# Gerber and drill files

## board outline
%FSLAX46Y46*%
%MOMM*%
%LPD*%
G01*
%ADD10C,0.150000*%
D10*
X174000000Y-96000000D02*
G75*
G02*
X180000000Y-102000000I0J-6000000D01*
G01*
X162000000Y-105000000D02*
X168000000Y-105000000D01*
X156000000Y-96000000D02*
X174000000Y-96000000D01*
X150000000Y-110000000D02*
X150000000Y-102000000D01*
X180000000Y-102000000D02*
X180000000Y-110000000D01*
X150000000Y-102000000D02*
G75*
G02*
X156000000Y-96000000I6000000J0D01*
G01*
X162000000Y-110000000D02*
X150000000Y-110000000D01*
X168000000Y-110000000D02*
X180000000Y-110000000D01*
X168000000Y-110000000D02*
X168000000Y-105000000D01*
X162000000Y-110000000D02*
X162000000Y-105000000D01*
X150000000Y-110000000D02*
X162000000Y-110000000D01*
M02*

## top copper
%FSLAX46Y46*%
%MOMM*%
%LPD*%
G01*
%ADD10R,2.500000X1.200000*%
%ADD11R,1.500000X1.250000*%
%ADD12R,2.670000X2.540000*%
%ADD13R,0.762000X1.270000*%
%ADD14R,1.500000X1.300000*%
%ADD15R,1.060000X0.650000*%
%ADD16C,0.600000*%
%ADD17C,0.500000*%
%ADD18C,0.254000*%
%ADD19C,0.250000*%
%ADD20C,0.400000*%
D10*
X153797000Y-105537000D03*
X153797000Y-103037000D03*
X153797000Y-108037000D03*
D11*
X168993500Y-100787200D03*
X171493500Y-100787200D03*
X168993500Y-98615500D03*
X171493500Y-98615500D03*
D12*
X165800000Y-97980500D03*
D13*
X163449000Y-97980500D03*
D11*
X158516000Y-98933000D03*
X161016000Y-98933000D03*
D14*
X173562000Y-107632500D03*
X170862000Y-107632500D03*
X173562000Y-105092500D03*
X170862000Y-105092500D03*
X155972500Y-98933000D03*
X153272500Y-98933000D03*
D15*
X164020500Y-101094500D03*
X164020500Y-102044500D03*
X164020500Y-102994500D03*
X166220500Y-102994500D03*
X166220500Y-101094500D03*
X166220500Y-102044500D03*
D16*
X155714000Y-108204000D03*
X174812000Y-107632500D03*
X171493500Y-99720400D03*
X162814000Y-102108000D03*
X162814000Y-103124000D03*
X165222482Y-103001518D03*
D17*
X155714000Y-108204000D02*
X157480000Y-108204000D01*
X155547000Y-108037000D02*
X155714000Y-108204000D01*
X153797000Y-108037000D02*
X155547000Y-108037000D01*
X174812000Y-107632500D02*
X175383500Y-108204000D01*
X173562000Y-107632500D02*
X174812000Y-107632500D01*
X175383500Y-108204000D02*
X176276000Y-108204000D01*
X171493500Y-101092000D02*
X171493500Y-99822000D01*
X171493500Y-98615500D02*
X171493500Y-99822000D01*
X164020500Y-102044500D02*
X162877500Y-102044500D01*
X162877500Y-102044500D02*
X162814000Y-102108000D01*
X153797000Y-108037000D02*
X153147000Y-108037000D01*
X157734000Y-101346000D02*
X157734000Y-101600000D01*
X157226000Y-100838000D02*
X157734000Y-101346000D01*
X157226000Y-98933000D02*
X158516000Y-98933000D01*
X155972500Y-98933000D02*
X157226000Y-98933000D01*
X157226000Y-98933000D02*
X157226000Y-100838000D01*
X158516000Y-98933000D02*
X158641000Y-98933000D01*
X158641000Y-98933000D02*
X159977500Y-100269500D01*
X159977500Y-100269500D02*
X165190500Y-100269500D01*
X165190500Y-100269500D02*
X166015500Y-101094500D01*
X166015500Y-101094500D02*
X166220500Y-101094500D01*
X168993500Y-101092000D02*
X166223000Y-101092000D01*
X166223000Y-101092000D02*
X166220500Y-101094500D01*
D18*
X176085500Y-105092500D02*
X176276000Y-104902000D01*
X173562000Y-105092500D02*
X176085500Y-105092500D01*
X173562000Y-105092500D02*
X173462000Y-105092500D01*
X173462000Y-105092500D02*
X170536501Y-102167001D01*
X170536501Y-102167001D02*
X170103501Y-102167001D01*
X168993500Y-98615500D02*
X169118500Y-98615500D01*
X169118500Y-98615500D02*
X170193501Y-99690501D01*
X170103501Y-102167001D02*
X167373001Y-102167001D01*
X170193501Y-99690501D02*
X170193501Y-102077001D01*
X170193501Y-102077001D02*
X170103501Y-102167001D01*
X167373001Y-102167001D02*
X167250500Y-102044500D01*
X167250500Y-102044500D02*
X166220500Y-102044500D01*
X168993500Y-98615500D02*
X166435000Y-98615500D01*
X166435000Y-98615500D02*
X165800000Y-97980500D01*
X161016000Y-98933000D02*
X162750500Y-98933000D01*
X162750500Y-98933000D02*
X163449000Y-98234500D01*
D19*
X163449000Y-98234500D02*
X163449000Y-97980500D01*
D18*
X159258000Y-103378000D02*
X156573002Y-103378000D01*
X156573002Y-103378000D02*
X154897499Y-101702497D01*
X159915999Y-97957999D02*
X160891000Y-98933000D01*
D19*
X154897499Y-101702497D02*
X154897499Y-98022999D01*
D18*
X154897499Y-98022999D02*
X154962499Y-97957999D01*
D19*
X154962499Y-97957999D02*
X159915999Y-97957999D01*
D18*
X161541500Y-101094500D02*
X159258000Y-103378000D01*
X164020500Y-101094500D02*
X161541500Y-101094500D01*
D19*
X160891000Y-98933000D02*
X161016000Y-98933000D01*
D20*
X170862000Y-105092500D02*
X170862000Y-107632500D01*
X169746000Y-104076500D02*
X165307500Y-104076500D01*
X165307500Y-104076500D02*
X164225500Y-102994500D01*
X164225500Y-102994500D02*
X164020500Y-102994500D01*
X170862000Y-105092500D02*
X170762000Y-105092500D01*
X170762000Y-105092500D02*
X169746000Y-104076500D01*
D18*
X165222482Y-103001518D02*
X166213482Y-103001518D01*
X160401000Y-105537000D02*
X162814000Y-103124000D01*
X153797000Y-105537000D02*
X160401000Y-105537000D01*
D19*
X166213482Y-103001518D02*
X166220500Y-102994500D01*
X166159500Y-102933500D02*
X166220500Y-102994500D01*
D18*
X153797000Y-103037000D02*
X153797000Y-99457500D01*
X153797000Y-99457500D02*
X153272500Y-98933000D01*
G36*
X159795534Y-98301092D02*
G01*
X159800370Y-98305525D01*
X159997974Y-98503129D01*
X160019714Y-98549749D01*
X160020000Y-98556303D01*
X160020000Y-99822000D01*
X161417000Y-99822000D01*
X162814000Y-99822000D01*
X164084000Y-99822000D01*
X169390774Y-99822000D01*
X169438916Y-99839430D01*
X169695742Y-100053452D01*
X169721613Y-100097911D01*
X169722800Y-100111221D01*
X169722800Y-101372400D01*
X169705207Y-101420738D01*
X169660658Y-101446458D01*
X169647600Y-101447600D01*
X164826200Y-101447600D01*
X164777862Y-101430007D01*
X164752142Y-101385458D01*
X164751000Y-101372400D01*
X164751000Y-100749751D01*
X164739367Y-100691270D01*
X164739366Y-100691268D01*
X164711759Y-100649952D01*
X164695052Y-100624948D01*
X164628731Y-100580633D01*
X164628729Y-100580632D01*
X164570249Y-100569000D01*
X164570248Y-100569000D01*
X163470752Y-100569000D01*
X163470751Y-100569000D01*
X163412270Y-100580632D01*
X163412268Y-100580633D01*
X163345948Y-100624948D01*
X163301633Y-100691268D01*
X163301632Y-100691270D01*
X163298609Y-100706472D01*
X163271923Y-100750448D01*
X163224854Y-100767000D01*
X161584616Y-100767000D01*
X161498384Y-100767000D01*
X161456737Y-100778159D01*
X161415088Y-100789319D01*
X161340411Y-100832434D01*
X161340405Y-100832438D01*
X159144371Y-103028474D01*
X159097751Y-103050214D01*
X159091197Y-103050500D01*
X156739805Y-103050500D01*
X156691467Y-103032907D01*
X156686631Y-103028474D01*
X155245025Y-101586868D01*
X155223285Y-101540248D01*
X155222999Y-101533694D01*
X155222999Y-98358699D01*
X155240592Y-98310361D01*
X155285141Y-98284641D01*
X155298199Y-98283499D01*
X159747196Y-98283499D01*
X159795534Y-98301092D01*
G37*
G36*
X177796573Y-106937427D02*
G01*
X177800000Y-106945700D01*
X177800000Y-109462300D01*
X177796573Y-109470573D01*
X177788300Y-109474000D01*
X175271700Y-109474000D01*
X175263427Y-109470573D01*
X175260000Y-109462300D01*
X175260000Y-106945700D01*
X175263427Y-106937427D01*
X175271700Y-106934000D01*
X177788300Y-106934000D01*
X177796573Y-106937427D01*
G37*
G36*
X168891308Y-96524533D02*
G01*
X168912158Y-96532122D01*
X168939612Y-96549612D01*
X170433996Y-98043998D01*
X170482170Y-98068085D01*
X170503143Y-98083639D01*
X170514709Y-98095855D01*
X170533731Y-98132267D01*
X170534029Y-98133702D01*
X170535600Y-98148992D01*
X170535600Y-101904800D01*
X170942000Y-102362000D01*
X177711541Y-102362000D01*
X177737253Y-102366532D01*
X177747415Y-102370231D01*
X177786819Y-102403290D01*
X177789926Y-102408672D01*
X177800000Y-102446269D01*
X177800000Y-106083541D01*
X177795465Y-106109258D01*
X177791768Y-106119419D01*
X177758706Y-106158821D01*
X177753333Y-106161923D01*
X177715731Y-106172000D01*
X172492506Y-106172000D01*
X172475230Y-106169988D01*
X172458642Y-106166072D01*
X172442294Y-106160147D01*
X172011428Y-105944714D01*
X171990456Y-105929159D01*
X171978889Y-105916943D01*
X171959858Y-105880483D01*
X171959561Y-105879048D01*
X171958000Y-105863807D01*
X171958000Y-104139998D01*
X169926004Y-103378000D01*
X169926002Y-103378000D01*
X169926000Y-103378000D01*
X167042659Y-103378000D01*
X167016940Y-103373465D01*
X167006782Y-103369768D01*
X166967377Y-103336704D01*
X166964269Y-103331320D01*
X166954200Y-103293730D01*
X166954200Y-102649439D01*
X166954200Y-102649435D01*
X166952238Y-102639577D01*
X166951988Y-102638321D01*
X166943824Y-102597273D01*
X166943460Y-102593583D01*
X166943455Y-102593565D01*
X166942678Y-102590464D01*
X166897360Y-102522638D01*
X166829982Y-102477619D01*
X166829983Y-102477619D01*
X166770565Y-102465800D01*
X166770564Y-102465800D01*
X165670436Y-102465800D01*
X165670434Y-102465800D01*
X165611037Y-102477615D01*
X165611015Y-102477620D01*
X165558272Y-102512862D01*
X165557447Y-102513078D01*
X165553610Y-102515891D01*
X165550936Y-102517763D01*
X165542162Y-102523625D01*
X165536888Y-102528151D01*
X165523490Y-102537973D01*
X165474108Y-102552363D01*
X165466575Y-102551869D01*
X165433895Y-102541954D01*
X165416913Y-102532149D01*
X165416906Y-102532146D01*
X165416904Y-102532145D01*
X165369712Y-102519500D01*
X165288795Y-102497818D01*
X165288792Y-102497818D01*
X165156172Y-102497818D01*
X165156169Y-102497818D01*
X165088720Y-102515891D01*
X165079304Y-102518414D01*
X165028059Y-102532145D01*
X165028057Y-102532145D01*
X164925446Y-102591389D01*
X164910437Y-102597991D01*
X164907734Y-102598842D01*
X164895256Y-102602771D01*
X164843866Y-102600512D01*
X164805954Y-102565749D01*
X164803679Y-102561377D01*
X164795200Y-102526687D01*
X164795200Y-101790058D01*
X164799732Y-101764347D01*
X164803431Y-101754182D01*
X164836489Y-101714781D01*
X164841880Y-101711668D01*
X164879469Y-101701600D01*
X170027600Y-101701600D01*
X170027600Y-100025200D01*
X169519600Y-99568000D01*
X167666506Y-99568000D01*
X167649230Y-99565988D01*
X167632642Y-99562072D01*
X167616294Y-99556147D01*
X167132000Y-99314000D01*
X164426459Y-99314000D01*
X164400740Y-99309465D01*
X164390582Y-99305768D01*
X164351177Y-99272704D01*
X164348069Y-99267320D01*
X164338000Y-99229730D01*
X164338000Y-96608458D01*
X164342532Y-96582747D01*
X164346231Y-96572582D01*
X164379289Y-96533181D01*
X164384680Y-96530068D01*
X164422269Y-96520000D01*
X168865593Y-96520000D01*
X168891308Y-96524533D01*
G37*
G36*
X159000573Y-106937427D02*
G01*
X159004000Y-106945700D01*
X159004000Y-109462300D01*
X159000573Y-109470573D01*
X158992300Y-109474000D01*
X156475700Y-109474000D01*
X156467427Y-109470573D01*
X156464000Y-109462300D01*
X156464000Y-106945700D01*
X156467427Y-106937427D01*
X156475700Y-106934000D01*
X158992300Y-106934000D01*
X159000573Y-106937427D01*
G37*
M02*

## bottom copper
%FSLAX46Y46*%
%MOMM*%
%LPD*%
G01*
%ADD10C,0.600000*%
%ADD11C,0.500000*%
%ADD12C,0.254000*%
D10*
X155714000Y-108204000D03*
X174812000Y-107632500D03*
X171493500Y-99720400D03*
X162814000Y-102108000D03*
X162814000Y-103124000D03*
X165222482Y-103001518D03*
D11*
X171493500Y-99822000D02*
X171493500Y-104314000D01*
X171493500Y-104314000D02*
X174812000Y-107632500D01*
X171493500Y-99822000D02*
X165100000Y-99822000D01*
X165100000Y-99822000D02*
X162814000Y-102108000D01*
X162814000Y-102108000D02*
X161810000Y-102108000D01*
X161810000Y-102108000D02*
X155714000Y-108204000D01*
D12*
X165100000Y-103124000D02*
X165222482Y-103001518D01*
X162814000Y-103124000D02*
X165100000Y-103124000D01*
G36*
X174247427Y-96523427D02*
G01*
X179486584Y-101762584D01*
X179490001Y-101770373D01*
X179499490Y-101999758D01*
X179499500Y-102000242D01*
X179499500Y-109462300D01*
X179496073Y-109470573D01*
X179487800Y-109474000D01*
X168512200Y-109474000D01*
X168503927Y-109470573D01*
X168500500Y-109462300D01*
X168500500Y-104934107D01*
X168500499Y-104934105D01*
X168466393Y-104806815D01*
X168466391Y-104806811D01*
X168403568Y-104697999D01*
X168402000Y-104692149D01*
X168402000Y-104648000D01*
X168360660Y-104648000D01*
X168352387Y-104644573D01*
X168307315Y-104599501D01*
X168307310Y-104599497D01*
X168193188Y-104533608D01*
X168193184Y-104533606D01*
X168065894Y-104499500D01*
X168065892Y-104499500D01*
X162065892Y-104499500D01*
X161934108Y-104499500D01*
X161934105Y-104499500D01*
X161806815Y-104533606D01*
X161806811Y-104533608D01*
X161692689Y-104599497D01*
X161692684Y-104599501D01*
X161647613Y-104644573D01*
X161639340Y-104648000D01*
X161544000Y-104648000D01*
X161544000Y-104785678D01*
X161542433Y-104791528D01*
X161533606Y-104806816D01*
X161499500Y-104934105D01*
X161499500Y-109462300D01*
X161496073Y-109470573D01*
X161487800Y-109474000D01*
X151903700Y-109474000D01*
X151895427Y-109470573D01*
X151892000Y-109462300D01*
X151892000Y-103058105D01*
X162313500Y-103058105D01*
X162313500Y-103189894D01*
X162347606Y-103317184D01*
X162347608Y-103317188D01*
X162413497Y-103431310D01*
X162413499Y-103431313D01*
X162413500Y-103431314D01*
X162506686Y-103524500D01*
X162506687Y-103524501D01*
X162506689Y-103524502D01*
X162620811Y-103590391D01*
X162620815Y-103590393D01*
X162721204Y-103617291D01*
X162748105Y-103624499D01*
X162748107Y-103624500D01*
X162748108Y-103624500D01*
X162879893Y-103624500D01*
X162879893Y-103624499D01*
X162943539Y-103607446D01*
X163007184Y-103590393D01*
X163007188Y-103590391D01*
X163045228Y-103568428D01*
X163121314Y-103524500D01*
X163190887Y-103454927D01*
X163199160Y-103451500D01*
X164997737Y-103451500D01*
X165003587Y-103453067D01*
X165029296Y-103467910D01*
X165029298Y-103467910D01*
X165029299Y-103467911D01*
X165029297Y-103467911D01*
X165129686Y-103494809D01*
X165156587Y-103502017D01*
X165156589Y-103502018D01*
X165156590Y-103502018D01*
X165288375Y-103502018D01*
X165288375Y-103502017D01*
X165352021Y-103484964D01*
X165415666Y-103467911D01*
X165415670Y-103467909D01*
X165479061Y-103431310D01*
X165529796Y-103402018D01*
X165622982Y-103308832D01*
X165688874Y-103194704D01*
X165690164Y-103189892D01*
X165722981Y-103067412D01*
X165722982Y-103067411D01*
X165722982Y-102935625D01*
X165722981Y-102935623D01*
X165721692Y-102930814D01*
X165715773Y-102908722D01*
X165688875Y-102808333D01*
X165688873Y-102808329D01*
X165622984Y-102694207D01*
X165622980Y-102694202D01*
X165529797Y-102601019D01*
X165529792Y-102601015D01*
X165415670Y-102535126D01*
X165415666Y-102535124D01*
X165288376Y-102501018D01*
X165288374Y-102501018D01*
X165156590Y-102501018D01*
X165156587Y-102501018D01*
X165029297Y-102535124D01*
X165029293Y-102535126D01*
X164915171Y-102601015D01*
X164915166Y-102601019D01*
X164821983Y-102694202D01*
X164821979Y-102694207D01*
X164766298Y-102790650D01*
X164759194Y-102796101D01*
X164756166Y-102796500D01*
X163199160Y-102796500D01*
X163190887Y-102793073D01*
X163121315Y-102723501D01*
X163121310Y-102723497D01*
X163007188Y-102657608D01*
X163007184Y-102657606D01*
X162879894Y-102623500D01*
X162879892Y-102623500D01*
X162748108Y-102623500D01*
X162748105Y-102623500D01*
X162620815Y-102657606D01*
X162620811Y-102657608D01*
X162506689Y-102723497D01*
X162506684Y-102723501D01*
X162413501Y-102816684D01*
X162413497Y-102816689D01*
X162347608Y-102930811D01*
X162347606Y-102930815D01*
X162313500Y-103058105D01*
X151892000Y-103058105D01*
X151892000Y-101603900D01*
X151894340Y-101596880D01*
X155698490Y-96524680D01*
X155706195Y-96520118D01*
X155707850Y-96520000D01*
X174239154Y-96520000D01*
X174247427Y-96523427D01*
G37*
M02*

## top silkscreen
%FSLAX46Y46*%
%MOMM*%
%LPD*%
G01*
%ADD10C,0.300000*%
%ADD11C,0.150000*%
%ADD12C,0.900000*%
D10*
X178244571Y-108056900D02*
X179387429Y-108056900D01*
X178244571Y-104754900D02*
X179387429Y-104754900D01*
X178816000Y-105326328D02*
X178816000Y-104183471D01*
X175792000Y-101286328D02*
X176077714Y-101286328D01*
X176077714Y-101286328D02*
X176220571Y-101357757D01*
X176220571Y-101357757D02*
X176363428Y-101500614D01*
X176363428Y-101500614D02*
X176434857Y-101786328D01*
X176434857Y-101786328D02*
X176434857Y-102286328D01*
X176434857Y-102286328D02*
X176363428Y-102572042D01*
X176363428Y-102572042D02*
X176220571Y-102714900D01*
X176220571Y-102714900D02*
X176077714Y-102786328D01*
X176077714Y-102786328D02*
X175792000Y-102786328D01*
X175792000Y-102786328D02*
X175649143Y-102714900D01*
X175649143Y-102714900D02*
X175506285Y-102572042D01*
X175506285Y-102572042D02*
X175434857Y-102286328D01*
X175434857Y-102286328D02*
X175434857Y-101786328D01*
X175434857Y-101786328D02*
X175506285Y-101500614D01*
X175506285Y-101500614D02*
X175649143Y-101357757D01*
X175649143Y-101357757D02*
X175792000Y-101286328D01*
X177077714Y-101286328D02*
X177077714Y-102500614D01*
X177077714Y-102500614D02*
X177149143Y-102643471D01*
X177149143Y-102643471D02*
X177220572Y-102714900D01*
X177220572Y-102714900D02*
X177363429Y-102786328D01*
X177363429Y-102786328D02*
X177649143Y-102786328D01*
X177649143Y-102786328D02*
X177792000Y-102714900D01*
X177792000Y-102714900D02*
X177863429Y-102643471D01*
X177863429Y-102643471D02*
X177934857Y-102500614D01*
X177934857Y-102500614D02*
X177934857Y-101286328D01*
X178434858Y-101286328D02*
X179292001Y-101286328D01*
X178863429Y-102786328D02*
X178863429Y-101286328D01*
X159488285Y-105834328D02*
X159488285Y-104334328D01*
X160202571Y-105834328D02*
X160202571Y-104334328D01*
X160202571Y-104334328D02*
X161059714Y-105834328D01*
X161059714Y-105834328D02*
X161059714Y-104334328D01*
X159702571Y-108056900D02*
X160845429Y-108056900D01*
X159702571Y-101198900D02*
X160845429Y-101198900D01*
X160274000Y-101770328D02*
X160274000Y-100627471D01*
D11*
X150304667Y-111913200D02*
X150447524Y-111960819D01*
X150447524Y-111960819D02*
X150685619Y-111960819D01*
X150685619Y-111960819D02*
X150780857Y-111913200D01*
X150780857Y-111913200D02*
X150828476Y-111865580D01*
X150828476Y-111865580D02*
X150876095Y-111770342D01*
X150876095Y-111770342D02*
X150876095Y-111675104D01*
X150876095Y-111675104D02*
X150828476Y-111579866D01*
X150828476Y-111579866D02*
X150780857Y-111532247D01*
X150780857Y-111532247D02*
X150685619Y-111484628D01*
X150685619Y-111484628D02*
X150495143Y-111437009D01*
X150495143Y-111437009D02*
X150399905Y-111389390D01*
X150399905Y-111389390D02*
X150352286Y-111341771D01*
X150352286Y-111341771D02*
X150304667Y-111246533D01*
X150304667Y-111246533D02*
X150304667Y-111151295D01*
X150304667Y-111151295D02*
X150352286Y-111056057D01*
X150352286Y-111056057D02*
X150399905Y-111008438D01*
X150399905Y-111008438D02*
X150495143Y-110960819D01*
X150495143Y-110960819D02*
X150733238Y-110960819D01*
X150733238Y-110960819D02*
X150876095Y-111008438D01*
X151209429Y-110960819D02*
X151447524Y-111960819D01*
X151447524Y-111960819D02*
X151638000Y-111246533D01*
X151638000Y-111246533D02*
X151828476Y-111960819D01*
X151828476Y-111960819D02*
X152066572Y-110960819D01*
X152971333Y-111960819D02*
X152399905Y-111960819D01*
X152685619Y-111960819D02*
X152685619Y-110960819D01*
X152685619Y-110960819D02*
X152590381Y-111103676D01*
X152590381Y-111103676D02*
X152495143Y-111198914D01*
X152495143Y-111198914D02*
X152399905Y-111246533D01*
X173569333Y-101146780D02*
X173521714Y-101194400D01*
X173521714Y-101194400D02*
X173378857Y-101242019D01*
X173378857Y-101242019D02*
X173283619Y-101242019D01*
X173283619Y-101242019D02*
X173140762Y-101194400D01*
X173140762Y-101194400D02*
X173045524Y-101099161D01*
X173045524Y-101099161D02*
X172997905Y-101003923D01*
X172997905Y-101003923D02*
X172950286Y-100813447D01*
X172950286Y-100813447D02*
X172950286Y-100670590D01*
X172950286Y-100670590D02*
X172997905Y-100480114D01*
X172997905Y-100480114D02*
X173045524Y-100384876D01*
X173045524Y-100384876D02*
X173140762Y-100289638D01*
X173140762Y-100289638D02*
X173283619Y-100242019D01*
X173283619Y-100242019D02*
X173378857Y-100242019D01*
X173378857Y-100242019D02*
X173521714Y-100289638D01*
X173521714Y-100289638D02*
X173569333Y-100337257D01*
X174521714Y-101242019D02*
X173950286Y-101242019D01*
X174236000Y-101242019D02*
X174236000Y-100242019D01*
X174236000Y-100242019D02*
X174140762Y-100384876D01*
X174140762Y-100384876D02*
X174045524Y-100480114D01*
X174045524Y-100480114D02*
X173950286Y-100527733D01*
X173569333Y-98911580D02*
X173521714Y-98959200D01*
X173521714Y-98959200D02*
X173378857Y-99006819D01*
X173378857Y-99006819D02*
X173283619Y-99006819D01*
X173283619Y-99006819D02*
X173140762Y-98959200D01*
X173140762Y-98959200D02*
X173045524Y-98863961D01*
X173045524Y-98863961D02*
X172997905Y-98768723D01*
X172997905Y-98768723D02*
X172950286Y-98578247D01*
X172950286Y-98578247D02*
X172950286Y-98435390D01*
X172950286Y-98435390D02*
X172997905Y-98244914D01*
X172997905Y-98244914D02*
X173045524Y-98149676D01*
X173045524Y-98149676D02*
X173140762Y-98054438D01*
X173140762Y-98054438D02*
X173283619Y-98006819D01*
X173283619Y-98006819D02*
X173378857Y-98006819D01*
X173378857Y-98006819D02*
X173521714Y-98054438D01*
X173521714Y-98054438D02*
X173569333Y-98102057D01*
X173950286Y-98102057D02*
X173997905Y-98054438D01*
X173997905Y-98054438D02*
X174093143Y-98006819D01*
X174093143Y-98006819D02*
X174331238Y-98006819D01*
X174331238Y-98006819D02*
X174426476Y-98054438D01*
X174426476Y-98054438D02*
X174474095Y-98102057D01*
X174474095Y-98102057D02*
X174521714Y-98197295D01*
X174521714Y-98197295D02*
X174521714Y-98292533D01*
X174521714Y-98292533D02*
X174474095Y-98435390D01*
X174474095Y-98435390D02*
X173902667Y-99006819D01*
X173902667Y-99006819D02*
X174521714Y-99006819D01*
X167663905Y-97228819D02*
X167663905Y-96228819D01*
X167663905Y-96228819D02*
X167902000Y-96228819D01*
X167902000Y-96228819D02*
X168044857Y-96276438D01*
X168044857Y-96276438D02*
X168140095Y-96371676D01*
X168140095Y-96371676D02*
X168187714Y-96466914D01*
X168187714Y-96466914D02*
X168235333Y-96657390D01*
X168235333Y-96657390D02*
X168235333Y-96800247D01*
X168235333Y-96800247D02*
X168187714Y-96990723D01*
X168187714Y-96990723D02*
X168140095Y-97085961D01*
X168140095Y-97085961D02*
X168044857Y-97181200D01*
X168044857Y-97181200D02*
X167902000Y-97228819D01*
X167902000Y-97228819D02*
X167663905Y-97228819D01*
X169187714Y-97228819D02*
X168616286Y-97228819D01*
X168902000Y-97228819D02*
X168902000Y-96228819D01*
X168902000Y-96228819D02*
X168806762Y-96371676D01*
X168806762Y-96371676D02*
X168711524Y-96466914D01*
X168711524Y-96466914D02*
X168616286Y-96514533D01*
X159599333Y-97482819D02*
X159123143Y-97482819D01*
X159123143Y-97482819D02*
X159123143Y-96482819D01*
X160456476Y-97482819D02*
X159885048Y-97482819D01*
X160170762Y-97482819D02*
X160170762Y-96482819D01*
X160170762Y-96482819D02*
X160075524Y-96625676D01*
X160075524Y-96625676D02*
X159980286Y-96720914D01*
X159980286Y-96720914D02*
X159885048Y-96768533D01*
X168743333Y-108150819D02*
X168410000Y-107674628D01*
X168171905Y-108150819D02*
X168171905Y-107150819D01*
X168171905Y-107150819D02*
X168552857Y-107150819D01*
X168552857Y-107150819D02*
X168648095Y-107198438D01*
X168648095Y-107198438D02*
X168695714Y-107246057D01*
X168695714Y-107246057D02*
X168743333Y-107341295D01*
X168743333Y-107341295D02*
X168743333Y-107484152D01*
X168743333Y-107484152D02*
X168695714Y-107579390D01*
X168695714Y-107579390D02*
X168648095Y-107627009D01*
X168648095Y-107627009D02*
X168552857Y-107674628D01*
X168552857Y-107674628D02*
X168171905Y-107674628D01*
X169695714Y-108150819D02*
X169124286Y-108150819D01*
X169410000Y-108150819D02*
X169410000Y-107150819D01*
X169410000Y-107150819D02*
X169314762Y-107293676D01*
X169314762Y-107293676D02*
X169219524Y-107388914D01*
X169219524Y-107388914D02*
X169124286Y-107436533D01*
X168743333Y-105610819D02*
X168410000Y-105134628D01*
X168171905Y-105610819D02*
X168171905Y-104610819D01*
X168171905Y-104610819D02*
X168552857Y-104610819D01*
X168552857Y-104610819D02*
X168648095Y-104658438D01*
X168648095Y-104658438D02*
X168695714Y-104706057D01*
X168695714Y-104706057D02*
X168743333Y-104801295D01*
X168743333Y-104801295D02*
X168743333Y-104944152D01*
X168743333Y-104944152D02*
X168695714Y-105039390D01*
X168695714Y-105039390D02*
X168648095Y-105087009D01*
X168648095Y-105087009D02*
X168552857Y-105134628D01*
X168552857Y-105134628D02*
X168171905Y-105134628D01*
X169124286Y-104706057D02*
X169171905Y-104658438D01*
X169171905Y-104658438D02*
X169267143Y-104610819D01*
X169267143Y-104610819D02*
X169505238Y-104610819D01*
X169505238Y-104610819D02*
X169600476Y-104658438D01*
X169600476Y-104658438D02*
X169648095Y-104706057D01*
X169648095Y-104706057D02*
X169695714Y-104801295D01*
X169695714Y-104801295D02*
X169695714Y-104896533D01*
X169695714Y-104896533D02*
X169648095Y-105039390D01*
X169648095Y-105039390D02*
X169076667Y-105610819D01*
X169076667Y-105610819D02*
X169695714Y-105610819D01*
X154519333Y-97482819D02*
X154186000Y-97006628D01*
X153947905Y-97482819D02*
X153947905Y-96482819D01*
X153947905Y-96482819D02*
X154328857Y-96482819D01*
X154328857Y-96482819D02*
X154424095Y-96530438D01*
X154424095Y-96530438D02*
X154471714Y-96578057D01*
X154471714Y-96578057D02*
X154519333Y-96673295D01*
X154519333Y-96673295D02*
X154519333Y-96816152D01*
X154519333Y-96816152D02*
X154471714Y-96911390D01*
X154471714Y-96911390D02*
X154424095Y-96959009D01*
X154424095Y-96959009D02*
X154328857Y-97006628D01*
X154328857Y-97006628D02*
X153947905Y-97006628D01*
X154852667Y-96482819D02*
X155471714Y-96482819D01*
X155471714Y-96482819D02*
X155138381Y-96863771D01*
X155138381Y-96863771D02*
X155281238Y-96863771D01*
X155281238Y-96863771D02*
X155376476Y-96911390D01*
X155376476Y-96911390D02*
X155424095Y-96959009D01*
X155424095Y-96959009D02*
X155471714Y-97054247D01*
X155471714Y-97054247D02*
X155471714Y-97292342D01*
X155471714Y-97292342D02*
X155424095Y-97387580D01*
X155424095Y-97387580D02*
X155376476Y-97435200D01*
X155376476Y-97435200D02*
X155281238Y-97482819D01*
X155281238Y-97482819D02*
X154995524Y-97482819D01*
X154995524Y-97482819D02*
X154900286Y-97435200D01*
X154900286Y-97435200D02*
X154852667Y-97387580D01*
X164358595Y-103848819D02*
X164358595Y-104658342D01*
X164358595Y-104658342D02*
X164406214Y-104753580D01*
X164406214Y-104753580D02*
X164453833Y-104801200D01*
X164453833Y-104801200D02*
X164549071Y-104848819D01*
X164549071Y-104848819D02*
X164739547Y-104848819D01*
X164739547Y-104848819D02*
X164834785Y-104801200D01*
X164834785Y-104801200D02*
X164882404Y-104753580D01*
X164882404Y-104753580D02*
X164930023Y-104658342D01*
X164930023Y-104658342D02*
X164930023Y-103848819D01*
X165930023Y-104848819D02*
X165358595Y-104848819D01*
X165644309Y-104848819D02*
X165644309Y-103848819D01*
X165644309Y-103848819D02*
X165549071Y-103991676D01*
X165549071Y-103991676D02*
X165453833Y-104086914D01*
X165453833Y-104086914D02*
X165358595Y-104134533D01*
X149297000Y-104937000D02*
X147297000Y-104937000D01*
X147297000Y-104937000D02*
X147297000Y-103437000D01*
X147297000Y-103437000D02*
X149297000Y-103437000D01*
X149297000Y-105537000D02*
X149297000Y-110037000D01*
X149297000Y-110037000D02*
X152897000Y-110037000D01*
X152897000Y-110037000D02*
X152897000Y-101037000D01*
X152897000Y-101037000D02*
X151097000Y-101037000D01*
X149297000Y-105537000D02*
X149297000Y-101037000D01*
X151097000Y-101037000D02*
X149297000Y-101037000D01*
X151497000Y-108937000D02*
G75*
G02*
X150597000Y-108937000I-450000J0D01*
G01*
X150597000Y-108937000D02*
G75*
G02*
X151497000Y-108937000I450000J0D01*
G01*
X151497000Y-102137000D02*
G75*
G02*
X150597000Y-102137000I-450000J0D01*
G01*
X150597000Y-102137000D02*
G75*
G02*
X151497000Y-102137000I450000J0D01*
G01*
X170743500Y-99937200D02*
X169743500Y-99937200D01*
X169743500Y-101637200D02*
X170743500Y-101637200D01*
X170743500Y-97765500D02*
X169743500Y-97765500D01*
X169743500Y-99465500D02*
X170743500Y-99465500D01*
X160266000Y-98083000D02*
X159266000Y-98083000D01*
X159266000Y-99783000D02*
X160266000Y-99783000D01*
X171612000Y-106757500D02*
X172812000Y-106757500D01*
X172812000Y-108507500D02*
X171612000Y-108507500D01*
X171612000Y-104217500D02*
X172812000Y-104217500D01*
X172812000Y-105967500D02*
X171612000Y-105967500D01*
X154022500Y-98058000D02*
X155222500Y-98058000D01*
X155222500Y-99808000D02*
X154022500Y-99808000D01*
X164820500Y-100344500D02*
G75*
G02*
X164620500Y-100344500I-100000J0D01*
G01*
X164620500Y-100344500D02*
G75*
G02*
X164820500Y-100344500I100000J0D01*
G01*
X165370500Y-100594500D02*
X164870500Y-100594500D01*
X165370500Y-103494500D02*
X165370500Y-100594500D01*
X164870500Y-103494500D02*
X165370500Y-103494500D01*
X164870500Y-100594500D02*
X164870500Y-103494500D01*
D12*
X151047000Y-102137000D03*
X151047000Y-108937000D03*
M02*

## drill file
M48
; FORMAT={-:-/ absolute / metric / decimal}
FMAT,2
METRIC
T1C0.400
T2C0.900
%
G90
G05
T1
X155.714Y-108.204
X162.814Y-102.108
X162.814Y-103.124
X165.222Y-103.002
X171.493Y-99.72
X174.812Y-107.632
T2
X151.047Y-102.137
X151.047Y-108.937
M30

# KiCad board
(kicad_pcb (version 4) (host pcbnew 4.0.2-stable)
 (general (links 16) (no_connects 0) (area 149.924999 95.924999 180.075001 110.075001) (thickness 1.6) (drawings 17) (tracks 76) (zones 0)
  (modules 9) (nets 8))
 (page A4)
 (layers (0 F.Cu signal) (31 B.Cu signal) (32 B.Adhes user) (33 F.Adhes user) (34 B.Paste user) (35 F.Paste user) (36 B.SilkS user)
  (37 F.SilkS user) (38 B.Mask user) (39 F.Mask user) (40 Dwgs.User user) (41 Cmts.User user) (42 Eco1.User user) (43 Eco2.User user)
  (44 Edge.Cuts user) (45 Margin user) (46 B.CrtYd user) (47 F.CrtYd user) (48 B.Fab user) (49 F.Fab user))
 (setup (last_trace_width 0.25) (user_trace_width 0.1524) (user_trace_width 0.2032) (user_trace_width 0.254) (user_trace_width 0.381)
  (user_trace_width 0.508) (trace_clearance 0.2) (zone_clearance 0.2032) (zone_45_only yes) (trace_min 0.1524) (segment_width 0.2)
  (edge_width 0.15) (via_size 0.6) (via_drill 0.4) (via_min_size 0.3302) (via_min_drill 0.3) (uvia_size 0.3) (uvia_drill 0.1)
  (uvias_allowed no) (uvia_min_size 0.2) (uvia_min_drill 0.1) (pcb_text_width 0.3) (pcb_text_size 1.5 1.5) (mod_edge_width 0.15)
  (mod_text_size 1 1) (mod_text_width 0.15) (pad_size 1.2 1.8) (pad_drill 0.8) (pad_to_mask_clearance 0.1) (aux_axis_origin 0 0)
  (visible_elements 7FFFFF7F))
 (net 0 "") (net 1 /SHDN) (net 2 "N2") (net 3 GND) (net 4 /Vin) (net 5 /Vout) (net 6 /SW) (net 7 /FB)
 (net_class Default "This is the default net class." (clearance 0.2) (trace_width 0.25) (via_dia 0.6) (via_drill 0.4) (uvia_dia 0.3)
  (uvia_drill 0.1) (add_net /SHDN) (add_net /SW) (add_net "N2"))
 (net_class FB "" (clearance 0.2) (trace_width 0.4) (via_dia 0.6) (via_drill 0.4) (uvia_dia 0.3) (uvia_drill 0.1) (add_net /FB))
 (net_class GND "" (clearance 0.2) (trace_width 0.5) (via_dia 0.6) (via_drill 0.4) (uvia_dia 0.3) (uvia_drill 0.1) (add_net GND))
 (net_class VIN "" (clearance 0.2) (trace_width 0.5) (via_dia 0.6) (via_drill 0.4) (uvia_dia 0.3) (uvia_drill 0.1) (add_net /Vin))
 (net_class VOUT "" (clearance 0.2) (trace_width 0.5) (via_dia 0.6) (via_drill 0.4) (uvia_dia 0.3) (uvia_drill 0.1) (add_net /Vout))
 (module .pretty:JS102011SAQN (layer F.Cu) (at 153.797 105.537 270)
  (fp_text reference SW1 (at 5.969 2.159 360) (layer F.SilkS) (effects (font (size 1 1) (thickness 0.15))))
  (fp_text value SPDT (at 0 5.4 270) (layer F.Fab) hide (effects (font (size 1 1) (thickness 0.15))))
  (fp_line (start -0.6 4.5) (end -0.6 6.5) (layer F.SilkS) (width 0.15))
  (fp_line (start -0.6 6.5) (end -2.1 6.5) (layer F.SilkS) (width 0.15))
  (fp_line (start -2.1 6.5) (end -2.1 4.5) (layer F.SilkS) (width 0.15))
  (fp_line (start 0 4.5) (end 4.5 4.5) (layer F.SilkS) (width 0.15))
  (fp_line (start 4.5 4.5) (end 4.5 0.9) (layer F.SilkS) (width 0.15))
  (fp_line (start 4.5 0.9) (end -4.5 0.9) (layer F.SilkS) (width 0.15))
  (fp_line (start -4.5 0.9) (end -4.5 2.7) (layer F.SilkS) (width 0.15))
  (fp_line (start 0 4.5) (end -4.5 4.5) (layer F.SilkS) (width 0.15))
  (fp_line (start -4.5 2.7) (end -4.5 4.5) (layer F.SilkS) (width 0.15))
  (fp_circle (center 3.4 2.75) (end 3.85 2.75) (layer F.SilkS) (width 0.15))
  (fp_circle (center -3.4 2.75) (end -3.85 2.75) (layer F.SilkS) (width 0.15))
  (pad 2 smd rect (at 0 0 270) (size 1.2 2.5) (layers F.Cu F.Paste F.Mask) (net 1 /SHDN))
  (pad 1 smd rect (at -2.5 0 270) (size 1.2 2.5) (layers F.Cu F.Paste F.Mask) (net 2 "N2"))
  (pad 3 smd rect (at 2.5 0 270) (size 1.2 2.5) (layers F.Cu F.Paste F.Mask) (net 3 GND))
  (pad "" np_thru_hole circle (at -3.4 2.75 270) (size 0.9 0.9) (drill 0.9) (layers *.Cu *.Mask F.SilkS))
  (pad "" np_thru_hole circle (at 3.4 2.75 270) (size 0.9 0.9) (drill 0.9) (layers *.Cu *.Mask F.SilkS)))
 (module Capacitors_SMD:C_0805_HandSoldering (layer F.Cu) (at 170.2435 100.7872)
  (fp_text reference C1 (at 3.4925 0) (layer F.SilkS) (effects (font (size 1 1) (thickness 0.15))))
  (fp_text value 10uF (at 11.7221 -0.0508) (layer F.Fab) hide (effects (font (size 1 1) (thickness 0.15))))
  (fp_line (start 0.5 -0.85) (end -0.5 -0.85) (layer F.SilkS) (width 0.15))
  (fp_line (start -0.5 0.85) (end 0.5 0.85) (layer F.SilkS) (width 0.15))
  (pad 1 smd rect (at -1.25 0) (size 1.5 1.25) (layers F.Cu F.Paste F.Mask) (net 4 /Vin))
  (pad 2 smd rect (at 1.25 0) (size 1.5 1.25) (layers F.Cu F.Paste F.Mask) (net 3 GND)))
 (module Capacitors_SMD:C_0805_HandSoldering (layer F.Cu) (at 170.2435 98.6155)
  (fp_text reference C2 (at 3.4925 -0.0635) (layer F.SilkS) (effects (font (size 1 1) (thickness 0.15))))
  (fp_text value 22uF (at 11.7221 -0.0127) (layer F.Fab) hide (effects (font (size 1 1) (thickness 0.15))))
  (fp_line (start 0.5 -0.85) (end -0.5 -0.85) (layer F.SilkS) (width 0.15))
  (fp_line (start -0.5 0.85) (end 0.5 0.85) (layer F.SilkS) (width 0.15))
  (pad 1 smd rect (at -1.25 0) (size 1.5 1.25) (layers F.Cu F.Paste F.Mask) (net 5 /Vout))
  (pad 2 smd rect (at 1.25 0) (size 1.5 1.25) (layers F.Cu F.Paste F.Mask) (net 3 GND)))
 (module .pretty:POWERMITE (layer F.Cu) (at 164.1475 97.9805 180)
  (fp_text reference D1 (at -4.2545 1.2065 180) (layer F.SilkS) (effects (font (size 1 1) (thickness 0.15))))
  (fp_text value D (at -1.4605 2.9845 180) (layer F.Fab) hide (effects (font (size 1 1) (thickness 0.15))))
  (pad 1 smd rect (at -1.6525 0 180) (size 2.67 2.54) (layers F.Cu F.Paste F.Mask) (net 5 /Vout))
  (pad 2 smd rect (at 0.6985 0 180) (size 0.762 1.27) (layers F.Cu F.Paste F.Mask) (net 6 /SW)))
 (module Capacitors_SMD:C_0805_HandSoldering (layer F.Cu) (at 159.766 98.933)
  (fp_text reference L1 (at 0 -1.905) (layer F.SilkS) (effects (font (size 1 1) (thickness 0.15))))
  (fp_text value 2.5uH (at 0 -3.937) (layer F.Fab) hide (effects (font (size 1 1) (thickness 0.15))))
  (fp_line (start 0.5 -0.85) (end -0.5 -0.85) (layer F.SilkS) (width 0.15))
  (fp_line (start -0.5 0.85) (end 0.5 0.85) (layer F.SilkS) (width 0.15))
  (pad 1 smd rect (at -1.25 0) (size 1.5 1.25) (layers F.Cu F.Paste F.Mask) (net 4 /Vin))
  (pad 2 smd rect (at 1.25 0) (size 1.5 1.25) (layers F.Cu F.Paste F.Mask) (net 6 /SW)))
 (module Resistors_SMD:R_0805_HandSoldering (layer F.Cu) (at 172.212 107.6325 180)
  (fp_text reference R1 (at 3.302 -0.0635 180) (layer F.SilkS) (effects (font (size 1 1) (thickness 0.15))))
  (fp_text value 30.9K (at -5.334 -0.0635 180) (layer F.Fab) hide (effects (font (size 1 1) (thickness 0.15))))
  (fp_line (start 0.6 0.875) (end -0.6 0.875) (layer F.SilkS) (width 0.15))
  (fp_line (start -0.6 -0.875) (end 0.6 -0.875) (layer F.SilkS) (width 0.15))
  (pad 1 smd rect (at -1.35 0 180) (size 1.5 1.3) (layers F.Cu F.Paste F.Mask) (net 3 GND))
  (pad 2 smd rect (at 1.35 0 180) (size 1.5 1.3) (layers F.Cu F.Paste F.Mask) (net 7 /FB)))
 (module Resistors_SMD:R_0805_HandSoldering (layer F.Cu) (at 172.212 105.0925 180)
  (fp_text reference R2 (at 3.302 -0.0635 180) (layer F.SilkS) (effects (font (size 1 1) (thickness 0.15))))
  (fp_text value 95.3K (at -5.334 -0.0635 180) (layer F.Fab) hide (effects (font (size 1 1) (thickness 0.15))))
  (fp_line (start 0.6 0.875) (end -0.6 0.875) (layer F.SilkS) (width 0.15))
  (fp_line (start -0.6 -0.875) (end 0.6 -0.875) (layer F.SilkS) (width 0.15))
  (pad 1 smd rect (at -1.35 0 180) (size 1.5 1.3) (layers F.Cu F.Paste F.Mask) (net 5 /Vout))
  (pad 2 smd rect (at 1.35 0 180) (size 1.5 1.3) (layers F.Cu F.Paste F.Mask) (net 7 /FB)))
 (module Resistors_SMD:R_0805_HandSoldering (layer F.Cu) (at 154.6225 98.933 180)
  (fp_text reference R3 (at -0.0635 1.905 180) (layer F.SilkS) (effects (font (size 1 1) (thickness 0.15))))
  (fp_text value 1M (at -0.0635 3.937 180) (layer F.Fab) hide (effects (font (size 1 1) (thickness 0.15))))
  (fp_line (start 0.6 0.875) (end -0.6 0.875) (layer F.SilkS) (width 0.15))
  (fp_line (start -0.6 -0.875) (end 0.6 -0.875) (layer F.SilkS) (width 0.15))
  (pad 1 smd rect (at -1.35 0 180) (size 1.5 1.3) (layers F.Cu F.Paste F.Mask) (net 4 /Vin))
  (pad 2 smd rect (at 1.35 0 180) (size 1.5 1.3) (layers F.Cu F.Paste F.Mask) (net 2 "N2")))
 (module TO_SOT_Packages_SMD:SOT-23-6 (layer F.Cu) (at 165.1205 102.0445)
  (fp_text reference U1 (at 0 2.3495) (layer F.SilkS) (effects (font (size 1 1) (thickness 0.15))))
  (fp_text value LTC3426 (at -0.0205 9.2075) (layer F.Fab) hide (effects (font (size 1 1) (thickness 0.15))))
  (fp_circle (center -0.4 -1.7) (end -0.3 -1.7) (layer F.SilkS) (width 0.15))
  (fp_line (start 0.25 -1.45) (end -0.25 -1.45) (layer F.SilkS) (width 0.15))
  (fp_line (start 0.25 1.45) (end 0.25 -1.45) (layer F.SilkS) (width 0.15))
  (fp_line (start -0.25 1.45) (end 0.25 1.45) (layer F.SilkS) (width 0.15))
  (fp_line (start -0.25 -1.45) (end -0.25 1.45) (layer F.SilkS) (width 0.15))
  (pad 1 smd rect (at -1.1 -0.95) (size 1.06 0.65) (layers F.Cu F.Paste F.Mask) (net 6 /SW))
  (pad 2 smd rect (at -1.1 0) (size 1.06 0.65) (layers F.Cu F.Paste F.Mask) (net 3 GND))
  (pad 3 smd rect (at -1.1 0.95) (size 1.06 0.65) (layers F.Cu F.Paste F.Mask) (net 7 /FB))
  (pad 4 smd rect (at 1.1 0.95) (size 1.06 0.65) (layers F.Cu F.Paste F.Mask) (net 1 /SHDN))
  (pad 6 smd rect (at 1.1 -0.95) (size 1.06 0.65) (layers F.Cu F.Paste F.Mask) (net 4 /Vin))
  (pad 5 smd rect (at 1.1 0) (size 1.06 0.65) (layers F.Cu F.Paste F.Mask) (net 5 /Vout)))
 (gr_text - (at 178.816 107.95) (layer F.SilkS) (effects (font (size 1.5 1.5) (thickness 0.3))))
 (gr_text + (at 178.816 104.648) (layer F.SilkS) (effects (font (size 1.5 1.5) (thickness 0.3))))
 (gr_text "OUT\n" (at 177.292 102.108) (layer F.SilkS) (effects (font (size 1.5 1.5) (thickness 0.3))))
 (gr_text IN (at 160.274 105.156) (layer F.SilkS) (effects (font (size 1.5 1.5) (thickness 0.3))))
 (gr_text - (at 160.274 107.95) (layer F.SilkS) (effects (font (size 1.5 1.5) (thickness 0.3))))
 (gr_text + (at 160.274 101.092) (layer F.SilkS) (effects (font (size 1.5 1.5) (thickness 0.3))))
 (gr_arc (start 174 102) (end 174 96) (angle 90) (layer Edge.Cuts) (width 0.15))
 (gr_line (start 162 105) (end 168 105) (angle 90) (layer Edge.Cuts) (width 0.15))
 (gr_line (start 156 96) (end 174 96) (angle 90) (layer Edge.Cuts) (width 0.15))
 (gr_line (start 150 110) (end 150 102) (angle 90) (layer Edge.Cuts) (width 0.15))
 (gr_line (start 180 102) (end 180 110) (angle 90) (layer Edge.Cuts) (width 0.15))
 (gr_arc (start 156 102) (end 150 102) (angle 90) (layer Edge.Cuts) (width 0.15))
 (gr_line (start 162 110) (end 150 110) (angle 90) (layer Edge.Cuts) (width 0.15))
 (gr_line (start 168 110) (end 180 110) (angle 90) (layer Edge.Cuts) (width 0.15))
 (gr_line (start 168 110) (end 168 105) (angle 90) (layer Edge.Cuts) (width 0.15))
 (gr_line (start 162 110) (end 162 105) (angle 90) (layer Edge.Cuts) (width 0.15))
 (gr_line (start 150 110) (end 162 110) (angle 90) (layer Edge.Cuts) (width 0.15))
 (segment (start 155.714 108.204) (end 157.48 108.204) (width 0.5) (layer F.Cu) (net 3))
 (via (at 155.714 108.204) (size 0.6) (drill 0.4) (layers F.Cu B.Cu) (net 3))
 (segment (start 155.547 108.037) (end 155.714 108.204) (width 0.5) (layer F.Cu) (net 3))
 (segment (start 153.797 108.037) (end 155.547 108.037) (width 0.5) (layer F.Cu) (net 3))
 (via (at 174.812 107.6325) (size 0.6) (drill 0.4) (layers F.Cu B.Cu) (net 3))
 (segment (start 174.812 107.6325) (end 175.3835 108.204) (width 0.5) (layer F.Cu) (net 3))
 (segment (start 173.562 107.6325) (end 174.812 107.6325) (width 0.5) (layer F.Cu) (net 3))
 (segment (start 175.3835 108.204) (end 176.276 108.204) (width 0.5) (layer F.Cu) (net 3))
 (segment (start 171.4935 99.822) (end 171.4935 104.314) (width 0.5) (layer B.Cu) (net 3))
 (segment (start 171.4935 104.314) (end 174.812 107.6325) (width 0.5) (layer B.Cu) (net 3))
 (segment (start 171.4935 99.822) (end 165.1 99.822) (width 0.5) (layer B.Cu) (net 3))
 (segment (start 165.1 99.822) (end 162.814 102.108) (width 0.5) (layer B.Cu) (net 3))
 (segment (start 162.814 102.108) (end 161.81 102.108) (width 0.5) (layer B.Cu) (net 3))
 (segment (start 161.81 102.108) (end 155.714 108.204) (width 0.5) (layer B.Cu) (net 3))
 (segment (start 171.4935 101.092) (end 171.4935 99.822) (width 0.5) (layer F.Cu) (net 3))
 (segment (start 171.4935 98.6155) (end 171.4935 99.822) (width 0.5) (layer F.Cu) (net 3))
 (via (at 171.4935 99.7204) (size 0.6) (drill 0.4) (layers F.Cu B.Cu) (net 3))
 (segment (start 164.0205 102.0445) (end 162.8775 102.0445) (width 0.5) (layer F.Cu) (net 3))
 (segment (start 162.8775 102.0445) (end 162.814 102.108) (width 0.5) (layer F.Cu) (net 3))
 (via (at 162.814 102.108) (size 0.6) (drill 0.4) (layers F.Cu B.Cu) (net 3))
 (segment (start 153.797 108.037) (end 153.147 108.037) (width 0.5) (layer F.Cu) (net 3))
 (segment (start 157.734 101.346) (end 157.734 101.6) (width 0.5) (layer F.Cu) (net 4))
 (segment (start 157.226 100.838) (end 157.734 101.346) (width 0.5) (layer F.Cu) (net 4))
 (segment (start 157.226 98.933) (end 158.516 98.933) (width 0.5) (layer F.Cu) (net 4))
 (segment (start 155.9725 98.933) (end 157.226 98.933) (width 0.5) (layer F.Cu) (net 4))
 (segment (start 157.226 98.933) (end 157.226 100.838) (width 0.5) (layer F.Cu) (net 4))
 (segment (start 158.516 98.933) (end 158.641 98.933) (width 0.5) (layer F.Cu) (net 4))
 (segment (start 158.641 98.933) (end 159.9775 100.2695) (width 0.5) (layer F.Cu) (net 4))
 (segment (start 159.9775 100.2695) (end 165.1905 100.2695) (width 0.5) (layer F.Cu) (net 4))
 (segment (start 165.1905 100.2695) (end 166.0155 101.0945) (width 0.5) (layer F.Cu) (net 4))
 (segment (start 166.0155 101.0945) (end 166.2205 101.0945) (width 0.5) (layer F.Cu) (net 4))
 (segment (start 168.9935 101.092) (end 166.223 101.092) (width 0.5) (layer F.Cu) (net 4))
 (segment (start 166.223 101.092) (end 166.2205 101.0945) (width 0.5) (layer F.Cu) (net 4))
 (segment (start 176.0855 105.0925) (end 176.276 104.902) (width 0.254) (layer F.Cu) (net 5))
 (segment (start 173.562 105.0925) (end 176.0855 105.0925) (width 0.254) (layer F.Cu) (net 5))
 (segment (start 173.562 105.0925) (end 173.462 105.0925) (width 0.254) (layer F.Cu) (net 5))
 (segment (start 173.462 105.0925) (end 170.536501 102.167001) (width 0.254) (layer F.Cu) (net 5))
 (segment (start 170.536501 102.167001) (end 170.103501 102.167001) (width 0.254) (layer F.Cu) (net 5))
 (segment (start 168.9935 98.6155) (end 169.1185 98.6155) (width 0.254) (layer F.Cu) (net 5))
 (segment (start 169.1185 98.6155) (end 170.193501 99.690501) (width 0.254) (layer F.Cu) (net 5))
 (segment (start 170.103501 102.167001) (end 167.373001 102.167001) (width 0.254) (layer F.Cu) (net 5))
 (segment (start 170.193501 99.690501) (end 170.193501 102.077001) (width 0.254) (layer F.Cu) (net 5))
 (segment (start 170.193501 102.077001) (end 170.103501 102.167001) (width 0.254) (layer F.Cu) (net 5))
 (segment (start 167.373001 102.167001) (end 167.2505 102.0445) (width 0.254) (layer F.Cu) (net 5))
 (segment (start 167.2505 102.0445) (end 166.2205 102.0445) (width 0.254) (layer F.Cu) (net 5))
 (segment (start 168.9935 98.6155) (end 166.435 98.6155) (width 0.254) (layer F.Cu) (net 5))
 (segment (start 166.435 98.6155) (end 165.8 97.9805) (width 0.254) (layer F.Cu) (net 5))
 (segment (start 161.016 98.933) (end 162.7505 98.933) (width 0.254) (layer F.Cu) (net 6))
 (segment (start 162.7505 98.933) (end 163.449 98.2345) (width 0.254) (layer F.Cu) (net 6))
 (segment (start 163.449 98.2345) (end 163.449 97.9805) (width 0.25) (layer F.Cu) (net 6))
 (segment (start 159.258 103.378) (end 156.573002 103.378) (width 0.254) (layer F.Cu) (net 6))
 (segment (start 156.573002 103.378) (end 154.897499 101.702497) (width 0.254) (layer F.Cu) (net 6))
 (segment (start 159.915999 97.957999) (end 160.891 98.933) (width 0.254) (layer F.Cu) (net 6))
 (segment (start 154.897499 101.702497) (end 154.897499 98.022999) (width 0.25) (layer F.Cu) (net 6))
 (segment (start 154.897499 98.022999) (end 154.962499 97.957999) (width 0.254) (layer F.Cu) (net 6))
 (segment (start 154.962499 97.957999) (end 159.915999 97.957999) (width 0.25) (layer F.Cu) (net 6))
 (segment (start 161.5415 101.0945) (end 159.258 103.378) (width 0.254) (layer F.Cu) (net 6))
 (segment (start 164.0205 101.0945) (end 161.5415 101.0945) (width 0.254) (layer F.Cu) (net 6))
 (segment (start 160.891 98.933) (end 161.016 98.933) (width 0.25) (layer F.Cu) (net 6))
 (segment (start 170.862 105.0925) (end 170.862 107.6325) (width 0.4) (layer F.Cu) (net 7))
 (segment (start 169.746 104.0765) (end 165.3075 104.0765) (width 0.4) (layer F.Cu) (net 7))
 (segment (start 165.3075 104.0765) (end 164.2255 102.9945) (width 0.4) (layer F.Cu) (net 7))
 (segment (start 164.2255 102.9945) (end 164.0205 102.9945) (width 0.4) (layer F.Cu) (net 7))
 (segment (start 170.862 105.0925) (end 170.762 105.0925) (width 0.4) (layer F.Cu) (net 7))
 (segment (start 170.762 105.0925) (end 169.746 104.0765) (width 0.4) (layer F.Cu) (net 7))
 (segment (start 165.222482 103.001518) (end 166.213482 103.001518) (width 0.254) (layer F.Cu) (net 1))
 (via (at 162.814 103.124) (size 0.6) (drill 0.4) (layers F.Cu B.Cu) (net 1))
 (segment (start 160.401 105.537) (end 162.814 103.124) (width 0.254) (layer F.Cu) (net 1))
 (segment (start 153.797 105.537) (end 160.401 105.537) (width 0.254) (layer F.Cu) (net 1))
 (via (at 165.222482 103.001518) (size 0.6) (drill 0.4) (layers F.Cu B.Cu) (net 1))
 (segment (start 165.1 103.124) (end 165.222482 103.001518) (width 0.254) (layer B.Cu) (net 1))
 (segment (start 162.814 103.124) (end 165.1 103.124) (width 0.254) (layer B.Cu) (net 1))
 (segment (start 166.213482 103.001518) (end 166.2205 102.9945) (width 0.25) (layer F.Cu) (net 1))
 (segment (start 166.1595 102.9335) (end 166.2205 102.9945) (width 0.25) (layer F.Cu) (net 1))
 (segment (start 153.797 103.037) (end 153.797 99.4575) (width 0.254) (layer F.Cu) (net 2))
 (segment (start 153.797 99.4575) (end 153.2725 98.933) (width 0.254) (layer F.Cu) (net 2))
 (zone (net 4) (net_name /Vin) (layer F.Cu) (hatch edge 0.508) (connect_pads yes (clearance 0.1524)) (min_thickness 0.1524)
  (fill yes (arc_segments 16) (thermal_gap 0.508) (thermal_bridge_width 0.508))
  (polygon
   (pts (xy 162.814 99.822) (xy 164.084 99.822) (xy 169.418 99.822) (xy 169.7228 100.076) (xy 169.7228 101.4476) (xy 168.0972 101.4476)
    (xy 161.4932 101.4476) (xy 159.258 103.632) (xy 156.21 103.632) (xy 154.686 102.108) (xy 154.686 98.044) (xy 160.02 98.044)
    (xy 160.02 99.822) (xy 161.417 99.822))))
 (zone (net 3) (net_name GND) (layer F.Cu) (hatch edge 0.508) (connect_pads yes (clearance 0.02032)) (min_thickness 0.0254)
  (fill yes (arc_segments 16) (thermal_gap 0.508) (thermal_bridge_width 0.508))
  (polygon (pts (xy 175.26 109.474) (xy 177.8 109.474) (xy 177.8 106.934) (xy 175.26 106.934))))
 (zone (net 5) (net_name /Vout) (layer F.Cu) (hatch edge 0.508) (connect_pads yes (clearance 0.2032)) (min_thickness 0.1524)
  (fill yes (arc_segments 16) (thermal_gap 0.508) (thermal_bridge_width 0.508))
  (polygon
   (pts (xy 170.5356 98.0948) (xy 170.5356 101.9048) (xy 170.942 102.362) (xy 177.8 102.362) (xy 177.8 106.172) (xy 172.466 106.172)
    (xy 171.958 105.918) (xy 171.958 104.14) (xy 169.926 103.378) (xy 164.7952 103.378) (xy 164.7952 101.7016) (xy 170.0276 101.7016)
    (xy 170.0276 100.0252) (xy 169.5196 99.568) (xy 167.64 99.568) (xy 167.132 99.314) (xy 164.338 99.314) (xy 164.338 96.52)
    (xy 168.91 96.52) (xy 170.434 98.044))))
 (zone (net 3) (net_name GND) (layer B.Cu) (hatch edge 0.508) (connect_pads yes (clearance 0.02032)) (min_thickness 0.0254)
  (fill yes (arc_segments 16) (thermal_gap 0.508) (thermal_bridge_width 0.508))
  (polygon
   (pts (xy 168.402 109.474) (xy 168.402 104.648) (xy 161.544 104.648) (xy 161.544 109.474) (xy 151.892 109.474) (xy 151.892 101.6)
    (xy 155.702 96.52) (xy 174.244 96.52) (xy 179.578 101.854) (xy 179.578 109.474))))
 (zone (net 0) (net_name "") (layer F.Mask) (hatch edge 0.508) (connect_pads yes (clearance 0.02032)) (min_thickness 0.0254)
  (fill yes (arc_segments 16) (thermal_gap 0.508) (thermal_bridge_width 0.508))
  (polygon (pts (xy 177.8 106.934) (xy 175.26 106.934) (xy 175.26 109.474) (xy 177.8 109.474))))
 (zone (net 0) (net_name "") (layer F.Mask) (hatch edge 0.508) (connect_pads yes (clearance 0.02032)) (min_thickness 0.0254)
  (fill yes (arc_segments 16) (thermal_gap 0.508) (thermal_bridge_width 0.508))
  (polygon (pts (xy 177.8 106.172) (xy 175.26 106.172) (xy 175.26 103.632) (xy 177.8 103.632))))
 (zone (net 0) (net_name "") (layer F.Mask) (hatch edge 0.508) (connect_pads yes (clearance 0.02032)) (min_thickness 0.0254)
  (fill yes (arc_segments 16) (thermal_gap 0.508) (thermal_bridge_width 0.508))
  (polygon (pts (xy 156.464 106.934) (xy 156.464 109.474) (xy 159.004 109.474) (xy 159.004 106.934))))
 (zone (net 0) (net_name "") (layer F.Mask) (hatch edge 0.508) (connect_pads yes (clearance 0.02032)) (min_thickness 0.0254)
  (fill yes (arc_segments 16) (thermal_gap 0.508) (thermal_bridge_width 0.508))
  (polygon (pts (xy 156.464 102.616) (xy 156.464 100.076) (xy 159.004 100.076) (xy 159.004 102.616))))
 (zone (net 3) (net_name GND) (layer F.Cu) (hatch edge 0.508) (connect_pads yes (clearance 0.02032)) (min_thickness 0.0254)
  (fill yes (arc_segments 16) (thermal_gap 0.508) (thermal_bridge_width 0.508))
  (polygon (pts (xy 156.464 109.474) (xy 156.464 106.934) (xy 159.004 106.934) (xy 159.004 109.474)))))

